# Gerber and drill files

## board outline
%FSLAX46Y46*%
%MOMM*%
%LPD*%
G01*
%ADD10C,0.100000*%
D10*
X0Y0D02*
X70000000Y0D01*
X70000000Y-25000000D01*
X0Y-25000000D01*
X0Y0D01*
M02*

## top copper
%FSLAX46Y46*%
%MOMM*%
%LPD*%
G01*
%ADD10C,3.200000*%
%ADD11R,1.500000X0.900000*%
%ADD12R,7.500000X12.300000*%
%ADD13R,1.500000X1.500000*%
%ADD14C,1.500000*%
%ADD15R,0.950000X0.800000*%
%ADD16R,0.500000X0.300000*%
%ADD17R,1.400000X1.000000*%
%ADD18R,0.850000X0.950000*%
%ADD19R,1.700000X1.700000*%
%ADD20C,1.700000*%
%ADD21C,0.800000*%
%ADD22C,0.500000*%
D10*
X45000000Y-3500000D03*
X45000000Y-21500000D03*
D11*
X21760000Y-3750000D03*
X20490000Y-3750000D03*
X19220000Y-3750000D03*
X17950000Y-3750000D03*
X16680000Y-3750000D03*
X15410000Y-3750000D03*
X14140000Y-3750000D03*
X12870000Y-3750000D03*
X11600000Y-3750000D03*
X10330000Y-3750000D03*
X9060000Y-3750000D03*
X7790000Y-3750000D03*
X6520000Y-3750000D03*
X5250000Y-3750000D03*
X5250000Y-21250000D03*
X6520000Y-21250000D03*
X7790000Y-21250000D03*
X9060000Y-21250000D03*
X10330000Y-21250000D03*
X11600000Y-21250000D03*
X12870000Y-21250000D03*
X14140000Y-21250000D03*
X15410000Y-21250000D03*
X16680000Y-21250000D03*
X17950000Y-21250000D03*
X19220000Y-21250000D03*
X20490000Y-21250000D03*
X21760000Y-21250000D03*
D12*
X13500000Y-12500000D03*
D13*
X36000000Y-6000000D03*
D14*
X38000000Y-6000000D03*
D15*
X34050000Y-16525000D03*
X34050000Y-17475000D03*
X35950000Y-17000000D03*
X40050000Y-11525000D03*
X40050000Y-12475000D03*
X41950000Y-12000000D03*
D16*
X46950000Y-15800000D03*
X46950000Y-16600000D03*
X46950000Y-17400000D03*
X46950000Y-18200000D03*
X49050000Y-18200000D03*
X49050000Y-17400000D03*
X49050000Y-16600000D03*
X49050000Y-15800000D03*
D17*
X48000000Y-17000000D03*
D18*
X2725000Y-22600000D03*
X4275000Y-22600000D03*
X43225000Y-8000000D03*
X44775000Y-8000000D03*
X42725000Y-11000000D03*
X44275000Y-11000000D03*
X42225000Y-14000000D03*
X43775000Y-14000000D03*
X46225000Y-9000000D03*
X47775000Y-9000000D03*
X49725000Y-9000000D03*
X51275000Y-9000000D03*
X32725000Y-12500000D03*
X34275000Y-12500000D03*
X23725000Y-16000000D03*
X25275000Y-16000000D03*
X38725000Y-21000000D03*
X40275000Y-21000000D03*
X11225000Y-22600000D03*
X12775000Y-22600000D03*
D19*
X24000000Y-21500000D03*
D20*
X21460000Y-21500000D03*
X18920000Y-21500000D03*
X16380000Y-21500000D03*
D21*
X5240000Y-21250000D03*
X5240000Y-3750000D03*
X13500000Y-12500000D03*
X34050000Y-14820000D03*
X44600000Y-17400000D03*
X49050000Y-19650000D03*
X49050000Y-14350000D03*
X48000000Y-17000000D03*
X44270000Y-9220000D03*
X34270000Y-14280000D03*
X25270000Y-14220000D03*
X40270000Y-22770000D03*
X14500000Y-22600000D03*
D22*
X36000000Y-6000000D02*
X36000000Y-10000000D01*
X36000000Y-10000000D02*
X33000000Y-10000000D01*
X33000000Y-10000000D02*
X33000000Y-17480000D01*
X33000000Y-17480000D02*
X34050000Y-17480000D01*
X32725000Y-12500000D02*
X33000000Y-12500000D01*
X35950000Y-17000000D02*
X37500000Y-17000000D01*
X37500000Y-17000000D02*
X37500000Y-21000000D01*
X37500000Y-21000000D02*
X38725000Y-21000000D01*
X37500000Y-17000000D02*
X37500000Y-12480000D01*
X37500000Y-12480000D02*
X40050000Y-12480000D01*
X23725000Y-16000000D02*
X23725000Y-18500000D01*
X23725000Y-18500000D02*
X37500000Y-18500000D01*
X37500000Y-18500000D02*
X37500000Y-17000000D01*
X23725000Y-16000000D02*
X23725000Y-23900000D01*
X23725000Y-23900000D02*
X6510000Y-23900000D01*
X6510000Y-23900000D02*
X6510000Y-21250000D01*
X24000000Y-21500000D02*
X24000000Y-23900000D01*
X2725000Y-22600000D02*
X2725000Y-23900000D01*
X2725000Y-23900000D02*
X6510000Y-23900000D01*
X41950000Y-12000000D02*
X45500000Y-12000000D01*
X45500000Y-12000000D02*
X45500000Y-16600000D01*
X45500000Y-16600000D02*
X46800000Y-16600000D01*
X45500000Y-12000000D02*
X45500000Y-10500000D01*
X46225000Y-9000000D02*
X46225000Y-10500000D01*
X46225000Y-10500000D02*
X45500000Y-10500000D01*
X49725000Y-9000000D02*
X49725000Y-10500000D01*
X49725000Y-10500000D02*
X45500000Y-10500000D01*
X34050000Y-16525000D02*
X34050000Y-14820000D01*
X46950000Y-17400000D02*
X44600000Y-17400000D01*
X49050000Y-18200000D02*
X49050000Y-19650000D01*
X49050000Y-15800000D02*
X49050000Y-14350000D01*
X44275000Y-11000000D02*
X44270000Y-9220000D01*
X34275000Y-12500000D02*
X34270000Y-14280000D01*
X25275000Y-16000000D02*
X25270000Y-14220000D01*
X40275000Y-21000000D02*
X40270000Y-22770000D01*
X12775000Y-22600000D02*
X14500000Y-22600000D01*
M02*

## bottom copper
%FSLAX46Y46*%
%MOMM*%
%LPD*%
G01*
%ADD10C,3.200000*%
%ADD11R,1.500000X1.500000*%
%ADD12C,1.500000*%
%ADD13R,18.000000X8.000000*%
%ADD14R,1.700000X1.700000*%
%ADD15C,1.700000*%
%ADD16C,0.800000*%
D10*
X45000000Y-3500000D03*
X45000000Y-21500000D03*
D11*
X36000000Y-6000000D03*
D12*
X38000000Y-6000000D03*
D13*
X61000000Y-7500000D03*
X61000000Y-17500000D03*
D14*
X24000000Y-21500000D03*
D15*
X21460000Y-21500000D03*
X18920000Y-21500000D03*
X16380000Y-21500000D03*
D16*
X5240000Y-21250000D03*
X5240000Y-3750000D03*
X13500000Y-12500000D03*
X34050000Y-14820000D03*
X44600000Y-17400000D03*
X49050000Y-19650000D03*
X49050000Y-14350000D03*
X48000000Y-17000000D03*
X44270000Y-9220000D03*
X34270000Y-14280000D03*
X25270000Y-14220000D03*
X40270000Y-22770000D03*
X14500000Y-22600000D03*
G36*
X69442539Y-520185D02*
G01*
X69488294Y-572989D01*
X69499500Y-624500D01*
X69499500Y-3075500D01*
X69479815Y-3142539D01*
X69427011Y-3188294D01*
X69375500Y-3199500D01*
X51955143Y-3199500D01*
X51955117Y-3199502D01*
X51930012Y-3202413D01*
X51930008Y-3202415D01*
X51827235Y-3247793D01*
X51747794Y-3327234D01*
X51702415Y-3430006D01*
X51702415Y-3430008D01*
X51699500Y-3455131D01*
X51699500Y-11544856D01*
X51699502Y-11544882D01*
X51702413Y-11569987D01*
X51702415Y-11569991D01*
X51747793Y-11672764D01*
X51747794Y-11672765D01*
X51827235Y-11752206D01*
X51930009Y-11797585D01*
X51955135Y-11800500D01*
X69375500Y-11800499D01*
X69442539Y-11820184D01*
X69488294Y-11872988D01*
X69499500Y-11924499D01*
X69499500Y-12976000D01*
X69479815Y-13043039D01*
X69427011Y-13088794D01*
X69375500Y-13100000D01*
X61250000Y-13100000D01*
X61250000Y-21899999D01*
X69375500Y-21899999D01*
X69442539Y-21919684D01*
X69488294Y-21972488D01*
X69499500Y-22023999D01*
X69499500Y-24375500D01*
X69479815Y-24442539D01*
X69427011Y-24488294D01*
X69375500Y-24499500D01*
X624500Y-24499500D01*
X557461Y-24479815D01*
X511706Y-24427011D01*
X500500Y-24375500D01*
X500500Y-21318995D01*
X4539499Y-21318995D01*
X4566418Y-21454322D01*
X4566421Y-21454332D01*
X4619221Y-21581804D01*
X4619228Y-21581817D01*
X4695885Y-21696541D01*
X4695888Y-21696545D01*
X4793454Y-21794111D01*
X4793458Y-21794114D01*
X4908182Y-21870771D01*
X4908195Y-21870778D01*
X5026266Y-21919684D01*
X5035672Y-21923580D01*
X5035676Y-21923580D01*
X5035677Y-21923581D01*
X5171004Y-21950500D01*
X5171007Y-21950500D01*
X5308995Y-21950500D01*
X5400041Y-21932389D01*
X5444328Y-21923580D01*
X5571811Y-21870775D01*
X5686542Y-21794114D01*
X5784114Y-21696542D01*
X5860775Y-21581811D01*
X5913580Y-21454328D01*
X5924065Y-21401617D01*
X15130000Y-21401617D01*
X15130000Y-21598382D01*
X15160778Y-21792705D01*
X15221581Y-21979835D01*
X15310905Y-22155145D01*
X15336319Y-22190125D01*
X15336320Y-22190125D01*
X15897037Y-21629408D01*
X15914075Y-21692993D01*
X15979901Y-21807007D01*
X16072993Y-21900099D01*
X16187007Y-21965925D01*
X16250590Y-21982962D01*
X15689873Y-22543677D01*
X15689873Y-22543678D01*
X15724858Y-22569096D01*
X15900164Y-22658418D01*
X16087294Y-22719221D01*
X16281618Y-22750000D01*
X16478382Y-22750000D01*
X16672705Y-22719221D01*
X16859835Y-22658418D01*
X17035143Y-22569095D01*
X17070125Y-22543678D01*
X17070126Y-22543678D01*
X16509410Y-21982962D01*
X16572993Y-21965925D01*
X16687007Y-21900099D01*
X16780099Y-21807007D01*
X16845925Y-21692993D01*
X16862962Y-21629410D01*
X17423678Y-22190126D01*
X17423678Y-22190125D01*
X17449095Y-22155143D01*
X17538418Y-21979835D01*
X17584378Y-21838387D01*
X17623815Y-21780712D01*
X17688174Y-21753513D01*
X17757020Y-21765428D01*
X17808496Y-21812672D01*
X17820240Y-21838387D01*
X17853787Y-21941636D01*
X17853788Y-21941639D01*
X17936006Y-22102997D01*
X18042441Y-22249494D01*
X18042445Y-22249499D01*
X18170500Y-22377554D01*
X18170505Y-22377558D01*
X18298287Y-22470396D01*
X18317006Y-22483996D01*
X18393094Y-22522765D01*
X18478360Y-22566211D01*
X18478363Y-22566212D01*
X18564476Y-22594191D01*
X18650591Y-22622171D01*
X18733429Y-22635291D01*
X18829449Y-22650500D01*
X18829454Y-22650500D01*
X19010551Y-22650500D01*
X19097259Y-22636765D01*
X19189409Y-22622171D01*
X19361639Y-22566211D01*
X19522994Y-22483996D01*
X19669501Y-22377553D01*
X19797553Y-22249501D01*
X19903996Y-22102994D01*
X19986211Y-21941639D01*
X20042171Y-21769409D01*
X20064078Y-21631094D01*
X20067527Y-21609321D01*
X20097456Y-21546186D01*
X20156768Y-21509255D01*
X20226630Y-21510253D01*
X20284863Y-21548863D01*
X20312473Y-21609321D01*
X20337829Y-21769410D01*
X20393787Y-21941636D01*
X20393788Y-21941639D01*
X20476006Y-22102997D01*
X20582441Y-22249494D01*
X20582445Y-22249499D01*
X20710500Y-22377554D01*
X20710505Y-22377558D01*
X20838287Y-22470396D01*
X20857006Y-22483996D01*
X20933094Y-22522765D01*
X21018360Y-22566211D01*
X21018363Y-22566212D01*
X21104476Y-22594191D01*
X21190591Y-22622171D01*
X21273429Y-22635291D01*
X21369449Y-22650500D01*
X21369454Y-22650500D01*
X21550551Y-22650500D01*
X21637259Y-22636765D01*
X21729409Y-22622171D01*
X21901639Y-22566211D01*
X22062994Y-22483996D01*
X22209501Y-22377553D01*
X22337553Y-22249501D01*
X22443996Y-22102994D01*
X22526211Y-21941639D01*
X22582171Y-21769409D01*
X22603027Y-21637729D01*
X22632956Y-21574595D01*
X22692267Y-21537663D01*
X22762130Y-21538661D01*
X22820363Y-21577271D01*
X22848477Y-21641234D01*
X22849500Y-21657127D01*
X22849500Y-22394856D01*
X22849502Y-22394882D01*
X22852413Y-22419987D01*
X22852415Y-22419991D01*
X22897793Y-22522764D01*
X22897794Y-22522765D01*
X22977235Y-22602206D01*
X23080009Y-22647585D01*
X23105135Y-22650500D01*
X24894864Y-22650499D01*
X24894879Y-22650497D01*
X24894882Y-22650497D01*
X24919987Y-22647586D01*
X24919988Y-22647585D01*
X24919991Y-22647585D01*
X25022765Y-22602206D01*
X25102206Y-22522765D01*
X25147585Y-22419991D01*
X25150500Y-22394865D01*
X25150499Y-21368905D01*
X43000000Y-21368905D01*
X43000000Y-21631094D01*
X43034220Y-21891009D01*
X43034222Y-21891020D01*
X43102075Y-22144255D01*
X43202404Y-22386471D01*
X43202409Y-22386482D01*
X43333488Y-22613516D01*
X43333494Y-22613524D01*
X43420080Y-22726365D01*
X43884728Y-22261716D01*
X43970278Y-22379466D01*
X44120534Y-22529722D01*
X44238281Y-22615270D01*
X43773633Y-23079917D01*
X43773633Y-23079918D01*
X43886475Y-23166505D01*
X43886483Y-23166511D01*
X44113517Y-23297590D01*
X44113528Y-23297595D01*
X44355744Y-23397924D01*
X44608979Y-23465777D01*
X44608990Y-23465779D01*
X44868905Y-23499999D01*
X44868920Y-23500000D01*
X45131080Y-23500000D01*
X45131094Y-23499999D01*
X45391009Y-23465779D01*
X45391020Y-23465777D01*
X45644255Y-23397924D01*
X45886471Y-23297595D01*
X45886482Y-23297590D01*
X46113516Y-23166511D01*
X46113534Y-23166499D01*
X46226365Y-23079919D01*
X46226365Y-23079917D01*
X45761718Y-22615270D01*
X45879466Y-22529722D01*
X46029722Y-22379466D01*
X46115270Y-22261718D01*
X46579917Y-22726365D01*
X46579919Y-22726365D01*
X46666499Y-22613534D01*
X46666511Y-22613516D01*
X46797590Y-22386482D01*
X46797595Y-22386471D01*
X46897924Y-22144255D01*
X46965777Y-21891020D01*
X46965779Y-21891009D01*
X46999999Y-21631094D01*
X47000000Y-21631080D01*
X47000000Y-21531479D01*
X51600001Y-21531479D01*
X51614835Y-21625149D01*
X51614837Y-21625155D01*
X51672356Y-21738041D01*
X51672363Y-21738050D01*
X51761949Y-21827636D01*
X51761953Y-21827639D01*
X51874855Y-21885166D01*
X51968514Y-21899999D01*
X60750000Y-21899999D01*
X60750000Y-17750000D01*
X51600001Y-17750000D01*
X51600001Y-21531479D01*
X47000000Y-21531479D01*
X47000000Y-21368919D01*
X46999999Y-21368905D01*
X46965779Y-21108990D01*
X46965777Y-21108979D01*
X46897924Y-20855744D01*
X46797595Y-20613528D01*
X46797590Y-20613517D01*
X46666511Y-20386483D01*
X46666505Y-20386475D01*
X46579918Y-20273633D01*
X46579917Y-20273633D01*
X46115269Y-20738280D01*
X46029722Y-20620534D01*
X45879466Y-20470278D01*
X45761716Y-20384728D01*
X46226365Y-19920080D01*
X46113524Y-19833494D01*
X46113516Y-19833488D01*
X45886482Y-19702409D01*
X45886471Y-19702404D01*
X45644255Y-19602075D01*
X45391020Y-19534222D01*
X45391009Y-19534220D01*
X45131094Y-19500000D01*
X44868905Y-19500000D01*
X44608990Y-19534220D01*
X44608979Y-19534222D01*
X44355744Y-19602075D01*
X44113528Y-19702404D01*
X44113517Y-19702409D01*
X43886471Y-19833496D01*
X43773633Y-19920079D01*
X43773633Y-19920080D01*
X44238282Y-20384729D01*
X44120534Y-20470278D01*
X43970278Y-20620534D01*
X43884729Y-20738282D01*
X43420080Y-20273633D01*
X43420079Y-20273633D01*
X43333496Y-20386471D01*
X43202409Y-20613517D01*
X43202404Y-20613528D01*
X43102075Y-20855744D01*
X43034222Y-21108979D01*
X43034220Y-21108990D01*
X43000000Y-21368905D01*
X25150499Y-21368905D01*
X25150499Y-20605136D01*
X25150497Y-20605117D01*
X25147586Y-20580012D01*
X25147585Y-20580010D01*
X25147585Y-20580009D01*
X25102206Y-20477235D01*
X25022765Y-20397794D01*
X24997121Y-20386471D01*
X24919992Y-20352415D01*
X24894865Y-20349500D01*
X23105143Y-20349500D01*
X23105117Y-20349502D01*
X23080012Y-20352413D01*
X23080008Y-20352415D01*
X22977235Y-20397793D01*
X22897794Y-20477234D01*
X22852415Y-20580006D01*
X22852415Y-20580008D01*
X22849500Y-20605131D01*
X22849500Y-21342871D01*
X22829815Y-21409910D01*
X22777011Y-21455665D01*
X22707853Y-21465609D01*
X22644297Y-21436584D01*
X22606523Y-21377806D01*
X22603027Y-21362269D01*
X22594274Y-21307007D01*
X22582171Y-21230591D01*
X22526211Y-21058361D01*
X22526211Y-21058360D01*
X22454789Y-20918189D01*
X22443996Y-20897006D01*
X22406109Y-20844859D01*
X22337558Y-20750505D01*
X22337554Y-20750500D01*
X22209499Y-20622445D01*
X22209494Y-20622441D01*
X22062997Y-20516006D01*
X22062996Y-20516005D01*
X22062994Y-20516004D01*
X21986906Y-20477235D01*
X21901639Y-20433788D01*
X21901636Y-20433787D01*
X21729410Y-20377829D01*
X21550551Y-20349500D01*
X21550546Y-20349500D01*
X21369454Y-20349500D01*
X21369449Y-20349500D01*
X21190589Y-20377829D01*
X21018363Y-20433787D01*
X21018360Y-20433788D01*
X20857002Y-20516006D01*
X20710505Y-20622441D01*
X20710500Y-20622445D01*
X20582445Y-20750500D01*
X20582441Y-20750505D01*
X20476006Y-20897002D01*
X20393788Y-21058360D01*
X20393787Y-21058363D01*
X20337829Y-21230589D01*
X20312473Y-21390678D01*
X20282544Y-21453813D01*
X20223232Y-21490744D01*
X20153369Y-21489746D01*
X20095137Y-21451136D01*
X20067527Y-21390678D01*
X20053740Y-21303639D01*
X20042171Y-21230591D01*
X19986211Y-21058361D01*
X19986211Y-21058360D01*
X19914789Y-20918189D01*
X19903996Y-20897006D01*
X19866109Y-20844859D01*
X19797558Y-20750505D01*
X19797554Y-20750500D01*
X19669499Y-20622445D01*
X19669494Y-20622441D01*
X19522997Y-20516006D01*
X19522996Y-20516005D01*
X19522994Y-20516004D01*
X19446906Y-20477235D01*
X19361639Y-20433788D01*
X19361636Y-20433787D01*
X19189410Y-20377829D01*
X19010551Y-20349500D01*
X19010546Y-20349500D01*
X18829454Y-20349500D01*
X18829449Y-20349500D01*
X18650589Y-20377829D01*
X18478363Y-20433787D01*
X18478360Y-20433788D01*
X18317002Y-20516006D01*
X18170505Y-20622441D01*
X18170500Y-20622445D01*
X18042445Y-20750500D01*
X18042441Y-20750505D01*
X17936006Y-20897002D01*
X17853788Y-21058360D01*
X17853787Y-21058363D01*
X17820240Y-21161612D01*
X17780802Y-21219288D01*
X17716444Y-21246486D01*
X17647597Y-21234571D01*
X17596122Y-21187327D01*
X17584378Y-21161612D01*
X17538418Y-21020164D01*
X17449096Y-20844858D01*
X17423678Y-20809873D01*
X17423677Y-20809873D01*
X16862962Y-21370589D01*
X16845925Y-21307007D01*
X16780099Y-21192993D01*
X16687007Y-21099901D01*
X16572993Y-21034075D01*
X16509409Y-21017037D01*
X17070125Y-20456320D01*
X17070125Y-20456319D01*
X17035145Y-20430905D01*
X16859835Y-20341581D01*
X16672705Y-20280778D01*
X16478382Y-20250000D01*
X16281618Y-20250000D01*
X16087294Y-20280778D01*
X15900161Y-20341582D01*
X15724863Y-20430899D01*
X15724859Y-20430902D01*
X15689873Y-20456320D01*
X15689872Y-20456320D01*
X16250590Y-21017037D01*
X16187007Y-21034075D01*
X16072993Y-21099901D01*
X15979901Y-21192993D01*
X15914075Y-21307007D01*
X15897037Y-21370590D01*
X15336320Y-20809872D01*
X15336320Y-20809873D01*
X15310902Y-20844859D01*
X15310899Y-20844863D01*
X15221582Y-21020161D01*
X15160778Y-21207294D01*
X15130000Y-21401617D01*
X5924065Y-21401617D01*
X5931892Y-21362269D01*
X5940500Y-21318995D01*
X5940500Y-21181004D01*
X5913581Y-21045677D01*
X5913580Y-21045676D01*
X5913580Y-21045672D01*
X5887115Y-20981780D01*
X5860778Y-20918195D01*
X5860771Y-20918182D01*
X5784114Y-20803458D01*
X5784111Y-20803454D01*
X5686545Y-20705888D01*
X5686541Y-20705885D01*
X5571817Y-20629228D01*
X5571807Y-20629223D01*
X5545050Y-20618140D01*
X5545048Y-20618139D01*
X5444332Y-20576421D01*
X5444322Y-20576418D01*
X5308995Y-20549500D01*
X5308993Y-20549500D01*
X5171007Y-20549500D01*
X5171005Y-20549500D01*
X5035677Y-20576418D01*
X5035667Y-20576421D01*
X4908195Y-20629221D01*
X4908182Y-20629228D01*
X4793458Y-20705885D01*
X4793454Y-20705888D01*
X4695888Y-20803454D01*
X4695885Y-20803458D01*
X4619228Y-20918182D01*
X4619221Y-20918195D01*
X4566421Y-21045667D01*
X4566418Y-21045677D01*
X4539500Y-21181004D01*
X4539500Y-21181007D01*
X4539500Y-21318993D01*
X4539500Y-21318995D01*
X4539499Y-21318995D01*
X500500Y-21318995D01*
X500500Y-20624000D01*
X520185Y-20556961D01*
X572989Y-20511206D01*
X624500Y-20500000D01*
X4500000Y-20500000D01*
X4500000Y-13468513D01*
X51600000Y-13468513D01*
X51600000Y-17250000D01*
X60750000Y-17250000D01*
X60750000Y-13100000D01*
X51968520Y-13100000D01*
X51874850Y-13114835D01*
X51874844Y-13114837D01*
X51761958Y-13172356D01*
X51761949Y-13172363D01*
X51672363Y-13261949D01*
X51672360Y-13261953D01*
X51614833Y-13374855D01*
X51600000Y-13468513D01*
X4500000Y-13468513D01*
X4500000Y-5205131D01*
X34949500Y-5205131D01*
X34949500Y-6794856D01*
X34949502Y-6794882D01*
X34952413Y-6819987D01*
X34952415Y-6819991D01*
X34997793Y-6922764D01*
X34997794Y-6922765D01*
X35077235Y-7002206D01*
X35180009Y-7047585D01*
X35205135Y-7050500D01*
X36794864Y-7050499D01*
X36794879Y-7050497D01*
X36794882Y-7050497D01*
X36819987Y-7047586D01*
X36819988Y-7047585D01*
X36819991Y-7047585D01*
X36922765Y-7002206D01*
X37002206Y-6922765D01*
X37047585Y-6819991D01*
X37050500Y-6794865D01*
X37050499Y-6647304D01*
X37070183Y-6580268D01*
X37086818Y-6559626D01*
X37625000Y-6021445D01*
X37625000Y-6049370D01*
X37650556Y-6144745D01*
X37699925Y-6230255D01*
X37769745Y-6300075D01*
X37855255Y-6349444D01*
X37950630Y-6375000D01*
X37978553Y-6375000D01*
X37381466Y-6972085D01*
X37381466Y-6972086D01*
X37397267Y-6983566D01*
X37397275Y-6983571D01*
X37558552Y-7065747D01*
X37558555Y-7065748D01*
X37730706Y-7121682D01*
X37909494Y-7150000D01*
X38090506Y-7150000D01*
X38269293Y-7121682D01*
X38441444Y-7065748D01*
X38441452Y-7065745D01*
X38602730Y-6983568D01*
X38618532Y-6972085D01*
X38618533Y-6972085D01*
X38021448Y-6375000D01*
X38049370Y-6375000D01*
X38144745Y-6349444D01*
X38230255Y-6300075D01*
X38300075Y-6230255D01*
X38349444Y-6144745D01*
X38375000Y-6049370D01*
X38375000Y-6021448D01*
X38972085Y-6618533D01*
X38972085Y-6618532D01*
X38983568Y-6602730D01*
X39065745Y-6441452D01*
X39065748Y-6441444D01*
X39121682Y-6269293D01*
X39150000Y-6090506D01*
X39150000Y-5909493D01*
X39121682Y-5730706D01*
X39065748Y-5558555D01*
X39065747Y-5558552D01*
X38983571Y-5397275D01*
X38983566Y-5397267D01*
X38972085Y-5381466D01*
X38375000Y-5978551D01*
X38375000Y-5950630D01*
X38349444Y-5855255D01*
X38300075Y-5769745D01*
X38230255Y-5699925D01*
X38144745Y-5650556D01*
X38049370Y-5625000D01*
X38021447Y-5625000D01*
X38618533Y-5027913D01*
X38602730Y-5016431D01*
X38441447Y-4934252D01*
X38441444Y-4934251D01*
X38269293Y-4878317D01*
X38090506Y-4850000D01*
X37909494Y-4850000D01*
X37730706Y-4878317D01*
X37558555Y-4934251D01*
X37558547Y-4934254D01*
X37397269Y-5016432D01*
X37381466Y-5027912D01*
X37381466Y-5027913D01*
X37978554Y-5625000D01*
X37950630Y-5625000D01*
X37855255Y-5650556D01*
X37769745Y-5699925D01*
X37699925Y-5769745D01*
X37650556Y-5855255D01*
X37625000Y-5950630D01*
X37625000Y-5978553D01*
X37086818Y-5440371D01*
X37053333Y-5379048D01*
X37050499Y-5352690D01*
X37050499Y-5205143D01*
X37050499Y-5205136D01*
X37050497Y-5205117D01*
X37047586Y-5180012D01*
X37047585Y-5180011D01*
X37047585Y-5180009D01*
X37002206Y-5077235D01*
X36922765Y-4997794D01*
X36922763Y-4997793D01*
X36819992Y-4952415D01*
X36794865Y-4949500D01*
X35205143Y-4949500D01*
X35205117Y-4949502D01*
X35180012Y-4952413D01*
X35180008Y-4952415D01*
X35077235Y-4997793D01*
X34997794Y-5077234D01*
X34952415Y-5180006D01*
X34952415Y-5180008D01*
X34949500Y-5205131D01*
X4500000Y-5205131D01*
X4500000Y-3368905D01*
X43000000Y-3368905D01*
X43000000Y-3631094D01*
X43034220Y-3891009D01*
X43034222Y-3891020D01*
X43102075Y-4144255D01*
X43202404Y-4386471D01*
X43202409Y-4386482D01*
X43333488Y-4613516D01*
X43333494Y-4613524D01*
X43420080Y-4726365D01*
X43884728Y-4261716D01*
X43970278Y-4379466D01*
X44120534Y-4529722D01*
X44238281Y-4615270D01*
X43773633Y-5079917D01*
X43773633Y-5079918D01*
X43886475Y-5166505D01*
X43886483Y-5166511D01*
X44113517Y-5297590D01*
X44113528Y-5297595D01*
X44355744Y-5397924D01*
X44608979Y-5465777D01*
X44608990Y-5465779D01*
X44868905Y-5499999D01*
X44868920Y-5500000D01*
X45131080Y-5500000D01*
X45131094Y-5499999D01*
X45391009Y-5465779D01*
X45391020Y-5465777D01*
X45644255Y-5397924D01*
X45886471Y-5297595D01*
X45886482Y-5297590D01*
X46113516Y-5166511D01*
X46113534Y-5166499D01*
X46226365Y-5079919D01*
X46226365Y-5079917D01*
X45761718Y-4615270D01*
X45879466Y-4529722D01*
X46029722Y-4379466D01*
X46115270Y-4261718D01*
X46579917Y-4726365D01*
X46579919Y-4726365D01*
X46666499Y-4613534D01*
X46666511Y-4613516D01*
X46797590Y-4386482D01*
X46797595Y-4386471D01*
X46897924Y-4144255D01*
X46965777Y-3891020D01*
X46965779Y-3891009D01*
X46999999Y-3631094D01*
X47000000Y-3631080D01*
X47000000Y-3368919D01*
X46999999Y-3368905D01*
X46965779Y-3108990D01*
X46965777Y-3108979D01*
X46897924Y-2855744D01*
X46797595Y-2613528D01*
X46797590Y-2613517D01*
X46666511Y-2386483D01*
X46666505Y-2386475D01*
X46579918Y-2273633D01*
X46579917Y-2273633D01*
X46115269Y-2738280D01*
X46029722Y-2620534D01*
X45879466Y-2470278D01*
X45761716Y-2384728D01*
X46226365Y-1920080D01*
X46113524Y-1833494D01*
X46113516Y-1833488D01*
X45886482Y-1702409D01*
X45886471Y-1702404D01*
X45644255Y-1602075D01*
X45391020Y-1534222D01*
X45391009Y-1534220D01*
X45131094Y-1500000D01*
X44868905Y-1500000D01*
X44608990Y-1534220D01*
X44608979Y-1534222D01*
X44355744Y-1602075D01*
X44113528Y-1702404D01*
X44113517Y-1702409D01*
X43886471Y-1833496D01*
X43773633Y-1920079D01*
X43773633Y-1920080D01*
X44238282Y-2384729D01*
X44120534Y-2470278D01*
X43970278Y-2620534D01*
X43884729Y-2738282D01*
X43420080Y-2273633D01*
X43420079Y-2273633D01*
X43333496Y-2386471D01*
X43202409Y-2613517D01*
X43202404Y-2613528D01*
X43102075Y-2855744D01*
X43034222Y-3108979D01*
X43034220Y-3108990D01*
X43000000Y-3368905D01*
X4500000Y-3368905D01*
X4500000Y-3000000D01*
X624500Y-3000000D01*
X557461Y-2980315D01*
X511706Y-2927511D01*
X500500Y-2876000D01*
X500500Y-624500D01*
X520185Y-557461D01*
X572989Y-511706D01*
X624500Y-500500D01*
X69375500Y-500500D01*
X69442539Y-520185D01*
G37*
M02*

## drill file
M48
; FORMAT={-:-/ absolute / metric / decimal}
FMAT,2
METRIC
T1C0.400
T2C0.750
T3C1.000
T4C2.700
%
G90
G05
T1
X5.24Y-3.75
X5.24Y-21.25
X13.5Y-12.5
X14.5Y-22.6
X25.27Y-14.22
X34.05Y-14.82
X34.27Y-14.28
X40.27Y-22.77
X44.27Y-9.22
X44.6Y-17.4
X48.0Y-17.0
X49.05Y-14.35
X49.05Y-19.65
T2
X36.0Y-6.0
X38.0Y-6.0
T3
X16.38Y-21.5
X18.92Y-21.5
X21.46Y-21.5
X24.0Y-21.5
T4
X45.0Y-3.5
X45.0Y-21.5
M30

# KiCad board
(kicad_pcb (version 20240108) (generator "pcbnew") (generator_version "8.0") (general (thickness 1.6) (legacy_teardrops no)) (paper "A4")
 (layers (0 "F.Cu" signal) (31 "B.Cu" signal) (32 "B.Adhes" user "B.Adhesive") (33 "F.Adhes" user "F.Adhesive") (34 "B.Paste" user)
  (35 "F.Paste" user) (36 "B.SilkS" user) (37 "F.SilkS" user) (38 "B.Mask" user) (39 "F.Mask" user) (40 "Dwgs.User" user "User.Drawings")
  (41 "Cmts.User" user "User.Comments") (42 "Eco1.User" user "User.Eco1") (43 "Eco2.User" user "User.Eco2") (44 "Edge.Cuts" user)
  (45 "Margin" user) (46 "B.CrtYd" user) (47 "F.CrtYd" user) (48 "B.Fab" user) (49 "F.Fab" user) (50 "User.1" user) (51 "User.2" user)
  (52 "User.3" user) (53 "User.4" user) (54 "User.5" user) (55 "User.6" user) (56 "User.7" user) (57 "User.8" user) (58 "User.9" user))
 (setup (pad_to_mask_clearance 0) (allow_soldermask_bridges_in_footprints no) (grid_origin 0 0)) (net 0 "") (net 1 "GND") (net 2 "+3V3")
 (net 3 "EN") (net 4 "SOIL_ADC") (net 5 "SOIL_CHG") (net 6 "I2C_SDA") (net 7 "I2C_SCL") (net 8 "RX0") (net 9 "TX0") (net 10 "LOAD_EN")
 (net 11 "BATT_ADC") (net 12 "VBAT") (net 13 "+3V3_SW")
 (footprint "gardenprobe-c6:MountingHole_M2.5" (layer "F.Cu") (at 45 3.5)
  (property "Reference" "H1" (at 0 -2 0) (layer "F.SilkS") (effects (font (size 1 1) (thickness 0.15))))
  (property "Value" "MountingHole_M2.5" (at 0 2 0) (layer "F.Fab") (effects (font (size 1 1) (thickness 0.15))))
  (pad "" np_thru_hole circle (at 0 0) (size 3.2 3.2) (drill 2.7) (layers "*.Cu" "*.Mask") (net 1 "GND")))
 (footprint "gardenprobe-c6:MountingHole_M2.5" (layer "F.Cu") (at 45 21.5)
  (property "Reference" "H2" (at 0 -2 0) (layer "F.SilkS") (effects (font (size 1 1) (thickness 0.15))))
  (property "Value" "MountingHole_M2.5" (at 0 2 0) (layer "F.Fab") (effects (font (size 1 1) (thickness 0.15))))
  (pad "" np_thru_hole circle (at 0 0) (size 3.2 3.2) (drill 2.7) (layers "*.Cu" "*.Mask") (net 1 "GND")))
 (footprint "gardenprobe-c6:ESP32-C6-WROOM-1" (layer "F.Cu") (at 13.5 12.5 270)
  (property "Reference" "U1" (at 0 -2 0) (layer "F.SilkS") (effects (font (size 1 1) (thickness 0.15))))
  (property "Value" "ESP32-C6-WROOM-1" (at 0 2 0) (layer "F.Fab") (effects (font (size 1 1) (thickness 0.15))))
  (pad "1" smd rect (at -8.75 -8.26) (size 1.5 0.9) (layers "F.Cu" "F.Paste" "F.Mask") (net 1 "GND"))
  (pad "2" smd rect (at -8.75 -6.99) (size 1.5 0.9) (layers "F.Cu" "F.Paste" "F.Mask") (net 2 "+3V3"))
  (pad "3" smd rect (at -8.75 -5.72) (size 1.5 0.9) (layers "F.Cu" "F.Paste" "F.Mask") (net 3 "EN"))
  (pad "4" smd rect (at -8.75 -4.45) (size 1.5 0.9) (layers "F.Cu" "F.Paste" "F.Mask"))
  (pad "5" smd rect (at -8.75 -3.18) (size 1.5 0.9) (layers "F.Cu" "F.Paste" "F.Mask"))
  (pad "6" smd rect (at -8.75 -1.91) (size 1.5 0.9) (layers "F.Cu" "F.Paste" "F.Mask"))
  (pad "7" smd rect (at -8.75 -0.64) (size 1.5 0.9) (layers "F.Cu" "F.Paste" "F.Mask"))
  (pad "8" smd rect (at -8.75 0.63) (size 1.5 0.9) (layers "F.Cu" "F.Paste" "F.Mask") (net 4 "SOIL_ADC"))
  (pad "9" smd rect (at -8.75 1.9) (size 1.5 0.9) (layers "F.Cu" "F.Paste" "F.Mask") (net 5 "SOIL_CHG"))
  (pad "10" smd rect (at -8.75 3.17) (size 1.5 0.9) (layers "F.Cu" "F.Paste" "F.Mask"))
  (pad "11" smd rect (at -8.75 4.44) (size 1.5 0.9) (layers "F.Cu" "F.Paste" "F.Mask"))
  (pad "12" smd rect (at -8.75 5.71) (size 1.5 0.9) (layers "F.Cu" "F.Paste" "F.Mask"))
  (pad "13" smd rect (at -8.75 6.98) (size 1.5 0.9) (layers "F.Cu" "F.Paste" "F.Mask"))
  (pad "14" smd rect (at -8.75 8.25) (size 1.5 0.9) (layers "F.Cu" "F.Paste" "F.Mask"))
  (pad "15" smd rect (at 8.75 8.25) (size 1.5 0.9) (layers "F.Cu" "F.Paste" "F.Mask"))
  (pad "16" smd rect (at 8.75 6.98) (size 1.5 0.9) (layers "F.Cu" "F.Paste" "F.Mask"))
  (pad "17" smd rect (at 8.75 5.71) (size 1.5 0.9) (layers "F.Cu" "F.Paste" "F.Mask"))
  (pad "18" smd rect (at 8.75 4.44) (size 1.5 0.9) (layers "F.Cu" "F.Paste" "F.Mask") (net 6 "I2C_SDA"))
  (pad "19" smd rect (at 8.75 3.17) (size 1.5 0.9) (layers "F.Cu" "F.Paste" "F.Mask") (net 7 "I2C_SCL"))
  (pad "20" smd rect (at 8.75 1.9) (size 1.5 0.9) (layers "F.Cu" "F.Paste" "F.Mask"))
  (pad "21" smd rect (at 8.75 0.63) (size 1.5 0.9) (layers "F.Cu" "F.Paste" "F.Mask"))
  (pad "22" smd rect (at 8.75 -0.64) (size 1.5 0.9) (layers "F.Cu" "F.Paste" "F.Mask"))
  (pad "23" smd rect (at 8.75 -1.91) (size 1.5 0.9) (layers "F.Cu" "F.Paste" "F.Mask"))
  (pad "24" smd rect (at 8.75 -3.18) (size 1.5 0.9) (layers "F.Cu" "F.Paste" "F.Mask") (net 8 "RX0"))
  (pad "25" smd rect (at 8.75 -4.45) (size 1.5 0.9) (layers "F.Cu" "F.Paste" "F.Mask") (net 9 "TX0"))
  (pad "26" smd rect (at 8.75 -5.72) (size 1.5 0.9) (layers "F.Cu" "F.Paste" "F.Mask") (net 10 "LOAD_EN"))
  (pad "27" smd rect (at 8.75 -6.99) (size 1.5 0.9) (layers "F.Cu" "F.Paste" "F.Mask") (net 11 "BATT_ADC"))
  (pad "28" smd rect (at 8.75 -8.26) (size 1.5 0.9) (layers "F.Cu" "F.Paste" "F.Mask") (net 1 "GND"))
  (pad "29" smd rect (at 0 0) (size 7.5 12.3) (layers "F.Cu" "F.Paste" "F.Mask") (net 1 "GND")))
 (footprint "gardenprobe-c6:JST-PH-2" (layer "F.Cu") (at 36 6)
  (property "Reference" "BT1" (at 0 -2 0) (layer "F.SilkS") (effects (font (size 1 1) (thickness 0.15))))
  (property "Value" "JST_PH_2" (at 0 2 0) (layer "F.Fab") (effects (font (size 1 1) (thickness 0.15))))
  (pad "1" thru_hole rect (at 0 0) (size 1.5 1.5) (drill 0.75) (layers "*.Cu" "*.Mask") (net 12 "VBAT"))
  (pad "2" thru_hole circle (at 2 0) (size 1.5 1.5) (drill 0.75) (layers "*.Cu" "*.Mask") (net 1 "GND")))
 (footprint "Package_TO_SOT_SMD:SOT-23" (layer "F.Cu") (at 35 17)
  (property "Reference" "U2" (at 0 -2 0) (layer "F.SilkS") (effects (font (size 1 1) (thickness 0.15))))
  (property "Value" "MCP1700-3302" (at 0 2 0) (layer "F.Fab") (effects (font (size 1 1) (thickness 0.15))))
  (pad "1" smd rect (at -0.95 -0.475) (size 0.95 0.8) (layers "F.Cu" "F.Paste" "F.Mask") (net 1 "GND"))
  (pad "2" smd rect (at -0.95 0.475) (size 0.95 0.8) (layers "F.Cu" "F.Paste" "F.Mask") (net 12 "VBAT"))
  (pad "3" smd rect (at 0.95 0) (size 0.95 0.8) (layers "F.Cu" "F.Paste" "F.Mask") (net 2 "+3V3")))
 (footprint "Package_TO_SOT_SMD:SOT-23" (layer "F.Cu") (at 41 12)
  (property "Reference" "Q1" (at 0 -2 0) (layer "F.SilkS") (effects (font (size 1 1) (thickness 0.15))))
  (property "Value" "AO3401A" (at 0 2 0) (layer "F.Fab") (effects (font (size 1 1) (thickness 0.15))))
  (pad "1" smd rect (at -0.95 -0.475) (size 0.95 0.8) (layers "F.Cu" "F.Paste" "F.Mask") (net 10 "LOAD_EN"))
  (pad "2" smd rect (at -0.95 0.475) (size 0.95 0.8) (layers "F.Cu" "F.Paste" "F.Mask") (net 2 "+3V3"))
  (pad "3" smd rect (at 0.95 0) (size 0.95 0.8) (layers "F.Cu" "F.Paste" "F.Mask") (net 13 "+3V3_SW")))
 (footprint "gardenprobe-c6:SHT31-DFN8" (layer "F.Cu") (at 48 17)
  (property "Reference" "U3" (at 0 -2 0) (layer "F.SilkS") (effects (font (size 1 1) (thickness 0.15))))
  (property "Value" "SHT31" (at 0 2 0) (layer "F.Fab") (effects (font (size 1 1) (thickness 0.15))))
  (pad "1" smd rect (at -1.05 -1.2) (size 0.5 0.3) (layers "F.Cu" "F.Paste" "F.Mask") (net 7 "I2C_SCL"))
  (pad "2" smd rect (at -1.05 -0.4) (size 0.5 0.3) (layers "F.Cu" "F.Paste" "F.Mask") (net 13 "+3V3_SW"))
  (pad "3" smd rect (at -1.05 0.4) (size 0.5 0.3) (layers "F.Cu" "F.Paste" "F.Mask") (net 1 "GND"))
  (pad "4" smd rect (at -1.05 1.2) (size 0.5 0.3) (layers "F.Cu" "F.Paste" "F.Mask") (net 6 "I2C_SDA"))
  (pad "8" smd rect (at 1.05 1.2) (size 0.5 0.3) (layers "F.Cu" "F.Paste" "F.Mask") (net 1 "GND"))
  (pad "7" smd rect (at 1.05 0.4) (size 0.5 0.3) (layers "F.Cu" "F.Paste" "F.Mask"))
  (pad "6" smd rect (at 1.05 -0.4) (size 0.5 0.3) (layers "F.Cu" "F.Paste" "F.Mask"))
  (pad "5" smd rect (at 1.05 -1.2) (size 0.5 0.3) (layers "F.Cu" "F.Paste" "F.Mask") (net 1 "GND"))
  (pad "9" smd rect (at 0 0) (size 1.4 1) (layers "F.Cu" "F.Paste" "F.Mask") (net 1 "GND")))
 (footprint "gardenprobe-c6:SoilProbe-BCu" (layer "F.Cu") (at 61 12.5)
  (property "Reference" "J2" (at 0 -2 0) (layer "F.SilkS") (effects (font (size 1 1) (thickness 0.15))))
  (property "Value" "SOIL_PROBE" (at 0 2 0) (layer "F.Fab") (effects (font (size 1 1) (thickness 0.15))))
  (pad "1" smd rect (at 0 -5) (size 18 8) (layers "B.Cu") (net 4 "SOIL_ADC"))
  (pad "2" smd rect (at 0 5) (size 18 8) (layers "B.Cu") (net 1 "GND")))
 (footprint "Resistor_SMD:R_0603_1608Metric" (layer "F.Cu") (at 3.5 22.6)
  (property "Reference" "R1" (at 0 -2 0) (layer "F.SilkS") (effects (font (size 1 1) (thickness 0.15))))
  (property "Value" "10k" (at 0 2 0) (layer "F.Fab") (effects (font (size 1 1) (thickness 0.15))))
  (pad "1" smd rect (at -0.775 0) (size 0.85 0.95) (layers "F.Cu" "F.Paste" "F.Mask") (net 2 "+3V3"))
  (pad "2" smd rect (at 0.775 0) (size 0.85 0.95) (layers "F.Cu" "F.Paste" "F.Mask") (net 3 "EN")))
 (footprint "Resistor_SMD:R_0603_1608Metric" (layer "F.Cu") (at 44 8)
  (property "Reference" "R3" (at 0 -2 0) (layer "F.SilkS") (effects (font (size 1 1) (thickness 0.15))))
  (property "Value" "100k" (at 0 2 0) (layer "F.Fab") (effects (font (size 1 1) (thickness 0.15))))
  (pad "1" smd rect (at -0.775 0) (size 0.85 0.95) (layers "F.Cu" "F.Paste" "F.Mask") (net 12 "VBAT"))
  (pad "2" smd rect (at 0.775 0) (size 0.85 0.95) (layers "F.Cu" "F.Paste" "F.Mask") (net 11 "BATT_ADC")))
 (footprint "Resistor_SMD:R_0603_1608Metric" (layer "F.Cu") (at 43.5 11)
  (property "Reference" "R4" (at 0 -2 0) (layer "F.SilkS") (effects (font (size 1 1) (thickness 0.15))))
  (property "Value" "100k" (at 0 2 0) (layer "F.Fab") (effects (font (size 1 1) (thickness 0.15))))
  (pad "1" smd rect (at -0.775 0) (size 0.85 0.95) (layers "F.Cu" "F.Paste" "F.Mask") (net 11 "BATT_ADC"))
  (pad "2" smd rect (at 0.775 0) (size 0.85 0.95) (layers "F.Cu" "F.Paste" "F.Mask") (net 1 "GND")))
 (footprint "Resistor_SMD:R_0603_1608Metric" (layer "F.Cu") (at 43 14)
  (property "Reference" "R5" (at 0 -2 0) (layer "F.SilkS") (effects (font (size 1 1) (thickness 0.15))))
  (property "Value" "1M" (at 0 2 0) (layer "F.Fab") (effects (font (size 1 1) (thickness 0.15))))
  (pad "1" smd rect (at -0.775 0) (size 0.85 0.95) (layers "F.Cu" "F.Paste" "F.Mask") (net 5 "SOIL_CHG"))
  (pad "2" smd rect (at 0.775 0) (size 0.85 0.95) (layers "F.Cu" "F.Paste" "F.Mask") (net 4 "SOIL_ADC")))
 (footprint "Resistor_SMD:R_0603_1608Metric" (layer "F.Cu") (at 47 9)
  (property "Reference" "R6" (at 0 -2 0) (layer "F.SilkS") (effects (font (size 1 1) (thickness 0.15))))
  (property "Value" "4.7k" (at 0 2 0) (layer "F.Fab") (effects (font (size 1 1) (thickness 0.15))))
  (pad "1" smd rect (at -0.775 0) (size 0.85 0.95) (layers "F.Cu" "F.Paste" "F.Mask") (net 13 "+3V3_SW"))
  (pad "2" smd rect (at 0.775 0) (size 0.85 0.95) (layers "F.Cu" "F.Paste" "F.Mask") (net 7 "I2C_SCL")))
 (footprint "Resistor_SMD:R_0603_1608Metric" (layer "F.Cu") (at 50.5 9)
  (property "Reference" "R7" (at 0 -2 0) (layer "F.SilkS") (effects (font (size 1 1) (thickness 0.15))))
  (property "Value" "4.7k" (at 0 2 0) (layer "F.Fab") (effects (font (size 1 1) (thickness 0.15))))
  (pad "1" smd rect (at -0.775 0) (size 0.85 0.95) (layers "F.Cu" "F.Paste" "F.Mask") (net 13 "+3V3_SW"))
  (pad "2" smd rect (at 0.775 0) (size 0.85 0.95) (layers "F.Cu" "F.Paste" "F.Mask") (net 6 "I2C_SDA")))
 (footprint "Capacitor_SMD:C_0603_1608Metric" (layer "F.Cu") (at 33.5 12.5)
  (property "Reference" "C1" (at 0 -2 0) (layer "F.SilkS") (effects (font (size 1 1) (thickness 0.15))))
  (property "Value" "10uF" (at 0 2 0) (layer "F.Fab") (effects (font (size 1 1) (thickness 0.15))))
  (pad "1" smd rect (at -0.775 0) (size 0.85 0.95) (layers "F.Cu" "F.Paste" "F.Mask") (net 12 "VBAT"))
  (pad "2" smd rect (at 0.775 0) (size 0.85 0.95) (layers "F.Cu" "F.Paste" "F.Mask") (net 1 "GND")))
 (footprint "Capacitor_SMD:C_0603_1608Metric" (layer "F.Cu") (at 24.5 16)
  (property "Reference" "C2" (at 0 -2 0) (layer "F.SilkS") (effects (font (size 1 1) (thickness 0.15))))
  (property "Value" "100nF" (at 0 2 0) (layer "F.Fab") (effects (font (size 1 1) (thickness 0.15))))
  (pad "1" smd rect (at -0.775 0) (size 0.85 0.95) (layers "F.Cu" "F.Paste" "F.Mask") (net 2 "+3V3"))
  (pad "2" smd rect (at 0.775 0) (size 0.85 0.95) (layers "F.Cu" "F.Paste" "F.Mask") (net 1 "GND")))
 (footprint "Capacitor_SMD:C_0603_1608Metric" (layer "F.Cu") (at 39.5 21)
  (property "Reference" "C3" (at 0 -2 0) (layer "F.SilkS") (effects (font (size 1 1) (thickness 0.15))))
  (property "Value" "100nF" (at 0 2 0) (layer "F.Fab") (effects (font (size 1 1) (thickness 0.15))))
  (pad "1" smd rect (at -0.775 0) (size 0.85 0.95) (layers "F.Cu" "F.Paste" "F.Mask") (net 2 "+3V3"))
  (pad "2" smd rect (at 0.775 0) (size 0.85 0.95) (layers "F.Cu" "F.Paste" "F.Mask") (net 1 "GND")))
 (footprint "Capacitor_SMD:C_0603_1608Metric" (layer "F.Cu") (at 12 22.6)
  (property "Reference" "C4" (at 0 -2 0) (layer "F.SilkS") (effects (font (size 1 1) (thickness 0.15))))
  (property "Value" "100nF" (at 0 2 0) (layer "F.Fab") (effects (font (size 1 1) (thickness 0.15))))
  (pad "1" smd rect (at -0.775 0) (size 0.85 0.95) (layers "F.Cu" "F.Paste" "F.Mask") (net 3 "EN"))
  (pad "2" smd rect (at 0.775 0) (size 0.85 0.95) (layers "F.Cu" "F.Paste" "F.Mask") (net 1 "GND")))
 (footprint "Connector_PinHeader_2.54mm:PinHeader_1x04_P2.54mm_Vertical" (layer "F.Cu") (at 24 21.5 270)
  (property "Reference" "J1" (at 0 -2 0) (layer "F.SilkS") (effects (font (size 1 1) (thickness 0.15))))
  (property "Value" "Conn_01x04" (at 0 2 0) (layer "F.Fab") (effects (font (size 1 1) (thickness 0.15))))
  (pad "1" thru_hole rect (at 0 0) (size 1.7 1.7) (drill 1) (layers "*.Cu" "*.Mask") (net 2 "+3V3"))
  (pad "2" thru_hole circle (at 0 2.54) (size 1.7 1.7) (drill 1) (layers "*.Cu" "*.Mask") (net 9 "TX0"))
  (pad "3" thru_hole circle (at 0 5.08) (size 1.7 1.7) (drill 1) (layers "*.Cu" "*.Mask") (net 8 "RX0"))
  (pad "4" thru_hole circle (at 0 7.62) (size 1.7 1.7) (drill 1) (layers "*.Cu" "*.Mask") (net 1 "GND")))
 (gr_rect (start 0 0) (end 70 25) (stroke (width 0.1) (type solid)) (fill none) (layer "Edge.Cuts"))
 (segment (start 36 6) (end 36 10) (width 0.5) (layer "F.Cu") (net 12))
 (segment (start 36 10) (end 33 10) (width 0.5) (layer "F.Cu") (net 12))
 (segment (start 33 10) (end 33 17.48) (width 0.5) (layer "F.Cu") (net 12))
 (segment (start 33 17.48) (end 34.05 17.48) (width 0.5) (layer "F.Cu") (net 12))
 (segment (start 32.725 12.5) (end 33 12.5) (width 0.5) (layer "F.Cu") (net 12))
 (segment (start 35.95 17) (end 37.5 17) (width 0.5) (layer "F.Cu") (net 2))
 (segment (start 37.5 17) (end 37.5 21) (width 0.5) (layer "F.Cu") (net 2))
 (segment (start 37.5 21) (end 38.725 21) (width 0.5) (layer "F.Cu") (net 2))
 (segment (start 37.5 17) (end 37.5 12.48) (width 0.5) (layer "F.Cu") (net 2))
 (segment (start 37.5 12.48) (end 40.05 12.48) (width 0.5) (layer "F.Cu") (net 2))
 (segment (start 23.725 16) (end 23.725 18.5) (width 0.5) (layer "F.Cu") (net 2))
 (segment (start 23.725 18.5) (end 37.5 18.5) (width 0.5) (layer "F.Cu") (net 2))
 (segment (start 37.5 18.5) (end 37.5 17) (width 0.5) (layer "F.Cu") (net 2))
 (segment (start 23.725 16) (end 23.725 23.9) (width 0.5) (layer "F.Cu") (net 2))
 (segment (start 23.725 23.9) (end 6.51 23.9) (width 0.5) (layer "F.Cu") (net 2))
 (segment (start 6.51 23.9) (end 6.51 21.25) (width 0.5) (layer "F.Cu") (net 2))
 (segment (start 24 21.5) (end 24 23.9) (width 0.5) (layer "F.Cu") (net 2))
 (segment (start 2.725 22.6) (end 2.725 23.9) (width 0.5) (layer "F.Cu") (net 2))
 (segment (start 2.725 23.9) (end 6.51 23.9) (width 0.5) (layer "F.Cu") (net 2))
 (segment (start 41.95 12) (end 45.5 12) (width 0.5) (layer "F.Cu") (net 13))
 (segment (start 45.5 12) (end 45.5 16.6) (width 0.5) (layer "F.Cu") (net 13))
 (segment (start 45.5 16.6) (end 46.8 16.6) (width 0.5) (layer "F.Cu") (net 13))
 (segment (start 45.5 12) (end 45.5 10.5) (width 0.5) (layer "F.Cu") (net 13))
 (segment (start 46.225 9) (end 46.225 10.5) (width 0.5) (layer "F.Cu") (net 13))
 (segment (start 46.225 10.5) (end 45.5 10.5) (width 0.5) (layer "F.Cu") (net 13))
 (segment (start 49.725 9) (end 49.725 10.5) (width 0.5) (layer "F.Cu") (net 13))
 (segment (start 49.725 10.5) (end 45.5 10.5) (width 0.5) (layer "F.Cu") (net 13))
 (segment (start 34.05 16.525) (end 34.05 14.82) (width 0.5) (layer "F.Cu") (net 1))
 (segment (start 46.95 17.4) (end 44.6 17.4) (width 0.5) (layer "F.Cu") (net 1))
 (segment (start 49.05 18.2) (end 49.05 19.65) (width 0.5) (layer "F.Cu") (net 1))
 (segment (start 49.05 15.8) (end 49.05 14.35) (width 0.5) (layer "F.Cu") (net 1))
 (segment (start 44.275 11) (end 44.27 9.22) (width 0.5) (layer "F.Cu") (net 1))
 (segment (start 34.275 12.5) (end 34.27 14.28) (width 0.5) (layer "F.Cu") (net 1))
 (segment (start 25.275 16) (end 25.27 14.22) (width 0.5) (layer "F.Cu") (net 1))
 (segment (start 40.275 21) (end 40.27 22.77) (width 0.5) (layer "F.Cu") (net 1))
 (segment (start 12.775 22.6) (end 14.5 22.6) (width 0.5) (layer "F.Cu") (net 1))
 (via (at 5.24 21.25) (size 0.8) (drill 0.4) (layers "F.Cu" "B.Cu") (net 1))
 (via (at 5.24 3.75) (size 0.8) (drill 0.4) (layers "F.Cu" "B.Cu") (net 1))
 (via (at 13.5 12.5) (size 0.8) (drill 0.4) (layers "F.Cu" "B.Cu") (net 1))
 (via (at 34.05 14.82) (size 0.8) (drill 0.4) (layers "F.Cu" "B.Cu") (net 1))
 (via (at 44.6 17.4) (size 0.8) (drill 0.4) (layers "F.Cu" "B.Cu") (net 1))
 (via (at 49.05 19.65) (size 0.8) (drill 0.4) (layers "F.Cu" "B.Cu") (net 1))
 (via (at 49.05 14.35) (size 0.8) (drill 0.4) (layers "F.Cu" "B.Cu") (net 1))
 (via (at 48 17) (size 0.8) (drill 0.4) (layers "F.Cu" "B.Cu") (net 1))
 (via (at 44.27 9.22) (size 0.8) (drill 0.4) (layers "F.Cu" "B.Cu") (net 1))
 (via (at 34.27 14.28) (size 0.8) (drill 0.4) (layers "F.Cu" "B.Cu") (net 1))
 (via (at 25.27 14.22) (size 0.8) (drill 0.4) (layers "F.Cu" "B.Cu") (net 1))
 (via (at 40.27 22.77) (size 0.8) (drill 0.4) (layers "F.Cu" "B.Cu") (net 1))
 (via (at 14.5 22.6) (size 0.8) (drill 0.4) (layers "F.Cu" "B.Cu") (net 1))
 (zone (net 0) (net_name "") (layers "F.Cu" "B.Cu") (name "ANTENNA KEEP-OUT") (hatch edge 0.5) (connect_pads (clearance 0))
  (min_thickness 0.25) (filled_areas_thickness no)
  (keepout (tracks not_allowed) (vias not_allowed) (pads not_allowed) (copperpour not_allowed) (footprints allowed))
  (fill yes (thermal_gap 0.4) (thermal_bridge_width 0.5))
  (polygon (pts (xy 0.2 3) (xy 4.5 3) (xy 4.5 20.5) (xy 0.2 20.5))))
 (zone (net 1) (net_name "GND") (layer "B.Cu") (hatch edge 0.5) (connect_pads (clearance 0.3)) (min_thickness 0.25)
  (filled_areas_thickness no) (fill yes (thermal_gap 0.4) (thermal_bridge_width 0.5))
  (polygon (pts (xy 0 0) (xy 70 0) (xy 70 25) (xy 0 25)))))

